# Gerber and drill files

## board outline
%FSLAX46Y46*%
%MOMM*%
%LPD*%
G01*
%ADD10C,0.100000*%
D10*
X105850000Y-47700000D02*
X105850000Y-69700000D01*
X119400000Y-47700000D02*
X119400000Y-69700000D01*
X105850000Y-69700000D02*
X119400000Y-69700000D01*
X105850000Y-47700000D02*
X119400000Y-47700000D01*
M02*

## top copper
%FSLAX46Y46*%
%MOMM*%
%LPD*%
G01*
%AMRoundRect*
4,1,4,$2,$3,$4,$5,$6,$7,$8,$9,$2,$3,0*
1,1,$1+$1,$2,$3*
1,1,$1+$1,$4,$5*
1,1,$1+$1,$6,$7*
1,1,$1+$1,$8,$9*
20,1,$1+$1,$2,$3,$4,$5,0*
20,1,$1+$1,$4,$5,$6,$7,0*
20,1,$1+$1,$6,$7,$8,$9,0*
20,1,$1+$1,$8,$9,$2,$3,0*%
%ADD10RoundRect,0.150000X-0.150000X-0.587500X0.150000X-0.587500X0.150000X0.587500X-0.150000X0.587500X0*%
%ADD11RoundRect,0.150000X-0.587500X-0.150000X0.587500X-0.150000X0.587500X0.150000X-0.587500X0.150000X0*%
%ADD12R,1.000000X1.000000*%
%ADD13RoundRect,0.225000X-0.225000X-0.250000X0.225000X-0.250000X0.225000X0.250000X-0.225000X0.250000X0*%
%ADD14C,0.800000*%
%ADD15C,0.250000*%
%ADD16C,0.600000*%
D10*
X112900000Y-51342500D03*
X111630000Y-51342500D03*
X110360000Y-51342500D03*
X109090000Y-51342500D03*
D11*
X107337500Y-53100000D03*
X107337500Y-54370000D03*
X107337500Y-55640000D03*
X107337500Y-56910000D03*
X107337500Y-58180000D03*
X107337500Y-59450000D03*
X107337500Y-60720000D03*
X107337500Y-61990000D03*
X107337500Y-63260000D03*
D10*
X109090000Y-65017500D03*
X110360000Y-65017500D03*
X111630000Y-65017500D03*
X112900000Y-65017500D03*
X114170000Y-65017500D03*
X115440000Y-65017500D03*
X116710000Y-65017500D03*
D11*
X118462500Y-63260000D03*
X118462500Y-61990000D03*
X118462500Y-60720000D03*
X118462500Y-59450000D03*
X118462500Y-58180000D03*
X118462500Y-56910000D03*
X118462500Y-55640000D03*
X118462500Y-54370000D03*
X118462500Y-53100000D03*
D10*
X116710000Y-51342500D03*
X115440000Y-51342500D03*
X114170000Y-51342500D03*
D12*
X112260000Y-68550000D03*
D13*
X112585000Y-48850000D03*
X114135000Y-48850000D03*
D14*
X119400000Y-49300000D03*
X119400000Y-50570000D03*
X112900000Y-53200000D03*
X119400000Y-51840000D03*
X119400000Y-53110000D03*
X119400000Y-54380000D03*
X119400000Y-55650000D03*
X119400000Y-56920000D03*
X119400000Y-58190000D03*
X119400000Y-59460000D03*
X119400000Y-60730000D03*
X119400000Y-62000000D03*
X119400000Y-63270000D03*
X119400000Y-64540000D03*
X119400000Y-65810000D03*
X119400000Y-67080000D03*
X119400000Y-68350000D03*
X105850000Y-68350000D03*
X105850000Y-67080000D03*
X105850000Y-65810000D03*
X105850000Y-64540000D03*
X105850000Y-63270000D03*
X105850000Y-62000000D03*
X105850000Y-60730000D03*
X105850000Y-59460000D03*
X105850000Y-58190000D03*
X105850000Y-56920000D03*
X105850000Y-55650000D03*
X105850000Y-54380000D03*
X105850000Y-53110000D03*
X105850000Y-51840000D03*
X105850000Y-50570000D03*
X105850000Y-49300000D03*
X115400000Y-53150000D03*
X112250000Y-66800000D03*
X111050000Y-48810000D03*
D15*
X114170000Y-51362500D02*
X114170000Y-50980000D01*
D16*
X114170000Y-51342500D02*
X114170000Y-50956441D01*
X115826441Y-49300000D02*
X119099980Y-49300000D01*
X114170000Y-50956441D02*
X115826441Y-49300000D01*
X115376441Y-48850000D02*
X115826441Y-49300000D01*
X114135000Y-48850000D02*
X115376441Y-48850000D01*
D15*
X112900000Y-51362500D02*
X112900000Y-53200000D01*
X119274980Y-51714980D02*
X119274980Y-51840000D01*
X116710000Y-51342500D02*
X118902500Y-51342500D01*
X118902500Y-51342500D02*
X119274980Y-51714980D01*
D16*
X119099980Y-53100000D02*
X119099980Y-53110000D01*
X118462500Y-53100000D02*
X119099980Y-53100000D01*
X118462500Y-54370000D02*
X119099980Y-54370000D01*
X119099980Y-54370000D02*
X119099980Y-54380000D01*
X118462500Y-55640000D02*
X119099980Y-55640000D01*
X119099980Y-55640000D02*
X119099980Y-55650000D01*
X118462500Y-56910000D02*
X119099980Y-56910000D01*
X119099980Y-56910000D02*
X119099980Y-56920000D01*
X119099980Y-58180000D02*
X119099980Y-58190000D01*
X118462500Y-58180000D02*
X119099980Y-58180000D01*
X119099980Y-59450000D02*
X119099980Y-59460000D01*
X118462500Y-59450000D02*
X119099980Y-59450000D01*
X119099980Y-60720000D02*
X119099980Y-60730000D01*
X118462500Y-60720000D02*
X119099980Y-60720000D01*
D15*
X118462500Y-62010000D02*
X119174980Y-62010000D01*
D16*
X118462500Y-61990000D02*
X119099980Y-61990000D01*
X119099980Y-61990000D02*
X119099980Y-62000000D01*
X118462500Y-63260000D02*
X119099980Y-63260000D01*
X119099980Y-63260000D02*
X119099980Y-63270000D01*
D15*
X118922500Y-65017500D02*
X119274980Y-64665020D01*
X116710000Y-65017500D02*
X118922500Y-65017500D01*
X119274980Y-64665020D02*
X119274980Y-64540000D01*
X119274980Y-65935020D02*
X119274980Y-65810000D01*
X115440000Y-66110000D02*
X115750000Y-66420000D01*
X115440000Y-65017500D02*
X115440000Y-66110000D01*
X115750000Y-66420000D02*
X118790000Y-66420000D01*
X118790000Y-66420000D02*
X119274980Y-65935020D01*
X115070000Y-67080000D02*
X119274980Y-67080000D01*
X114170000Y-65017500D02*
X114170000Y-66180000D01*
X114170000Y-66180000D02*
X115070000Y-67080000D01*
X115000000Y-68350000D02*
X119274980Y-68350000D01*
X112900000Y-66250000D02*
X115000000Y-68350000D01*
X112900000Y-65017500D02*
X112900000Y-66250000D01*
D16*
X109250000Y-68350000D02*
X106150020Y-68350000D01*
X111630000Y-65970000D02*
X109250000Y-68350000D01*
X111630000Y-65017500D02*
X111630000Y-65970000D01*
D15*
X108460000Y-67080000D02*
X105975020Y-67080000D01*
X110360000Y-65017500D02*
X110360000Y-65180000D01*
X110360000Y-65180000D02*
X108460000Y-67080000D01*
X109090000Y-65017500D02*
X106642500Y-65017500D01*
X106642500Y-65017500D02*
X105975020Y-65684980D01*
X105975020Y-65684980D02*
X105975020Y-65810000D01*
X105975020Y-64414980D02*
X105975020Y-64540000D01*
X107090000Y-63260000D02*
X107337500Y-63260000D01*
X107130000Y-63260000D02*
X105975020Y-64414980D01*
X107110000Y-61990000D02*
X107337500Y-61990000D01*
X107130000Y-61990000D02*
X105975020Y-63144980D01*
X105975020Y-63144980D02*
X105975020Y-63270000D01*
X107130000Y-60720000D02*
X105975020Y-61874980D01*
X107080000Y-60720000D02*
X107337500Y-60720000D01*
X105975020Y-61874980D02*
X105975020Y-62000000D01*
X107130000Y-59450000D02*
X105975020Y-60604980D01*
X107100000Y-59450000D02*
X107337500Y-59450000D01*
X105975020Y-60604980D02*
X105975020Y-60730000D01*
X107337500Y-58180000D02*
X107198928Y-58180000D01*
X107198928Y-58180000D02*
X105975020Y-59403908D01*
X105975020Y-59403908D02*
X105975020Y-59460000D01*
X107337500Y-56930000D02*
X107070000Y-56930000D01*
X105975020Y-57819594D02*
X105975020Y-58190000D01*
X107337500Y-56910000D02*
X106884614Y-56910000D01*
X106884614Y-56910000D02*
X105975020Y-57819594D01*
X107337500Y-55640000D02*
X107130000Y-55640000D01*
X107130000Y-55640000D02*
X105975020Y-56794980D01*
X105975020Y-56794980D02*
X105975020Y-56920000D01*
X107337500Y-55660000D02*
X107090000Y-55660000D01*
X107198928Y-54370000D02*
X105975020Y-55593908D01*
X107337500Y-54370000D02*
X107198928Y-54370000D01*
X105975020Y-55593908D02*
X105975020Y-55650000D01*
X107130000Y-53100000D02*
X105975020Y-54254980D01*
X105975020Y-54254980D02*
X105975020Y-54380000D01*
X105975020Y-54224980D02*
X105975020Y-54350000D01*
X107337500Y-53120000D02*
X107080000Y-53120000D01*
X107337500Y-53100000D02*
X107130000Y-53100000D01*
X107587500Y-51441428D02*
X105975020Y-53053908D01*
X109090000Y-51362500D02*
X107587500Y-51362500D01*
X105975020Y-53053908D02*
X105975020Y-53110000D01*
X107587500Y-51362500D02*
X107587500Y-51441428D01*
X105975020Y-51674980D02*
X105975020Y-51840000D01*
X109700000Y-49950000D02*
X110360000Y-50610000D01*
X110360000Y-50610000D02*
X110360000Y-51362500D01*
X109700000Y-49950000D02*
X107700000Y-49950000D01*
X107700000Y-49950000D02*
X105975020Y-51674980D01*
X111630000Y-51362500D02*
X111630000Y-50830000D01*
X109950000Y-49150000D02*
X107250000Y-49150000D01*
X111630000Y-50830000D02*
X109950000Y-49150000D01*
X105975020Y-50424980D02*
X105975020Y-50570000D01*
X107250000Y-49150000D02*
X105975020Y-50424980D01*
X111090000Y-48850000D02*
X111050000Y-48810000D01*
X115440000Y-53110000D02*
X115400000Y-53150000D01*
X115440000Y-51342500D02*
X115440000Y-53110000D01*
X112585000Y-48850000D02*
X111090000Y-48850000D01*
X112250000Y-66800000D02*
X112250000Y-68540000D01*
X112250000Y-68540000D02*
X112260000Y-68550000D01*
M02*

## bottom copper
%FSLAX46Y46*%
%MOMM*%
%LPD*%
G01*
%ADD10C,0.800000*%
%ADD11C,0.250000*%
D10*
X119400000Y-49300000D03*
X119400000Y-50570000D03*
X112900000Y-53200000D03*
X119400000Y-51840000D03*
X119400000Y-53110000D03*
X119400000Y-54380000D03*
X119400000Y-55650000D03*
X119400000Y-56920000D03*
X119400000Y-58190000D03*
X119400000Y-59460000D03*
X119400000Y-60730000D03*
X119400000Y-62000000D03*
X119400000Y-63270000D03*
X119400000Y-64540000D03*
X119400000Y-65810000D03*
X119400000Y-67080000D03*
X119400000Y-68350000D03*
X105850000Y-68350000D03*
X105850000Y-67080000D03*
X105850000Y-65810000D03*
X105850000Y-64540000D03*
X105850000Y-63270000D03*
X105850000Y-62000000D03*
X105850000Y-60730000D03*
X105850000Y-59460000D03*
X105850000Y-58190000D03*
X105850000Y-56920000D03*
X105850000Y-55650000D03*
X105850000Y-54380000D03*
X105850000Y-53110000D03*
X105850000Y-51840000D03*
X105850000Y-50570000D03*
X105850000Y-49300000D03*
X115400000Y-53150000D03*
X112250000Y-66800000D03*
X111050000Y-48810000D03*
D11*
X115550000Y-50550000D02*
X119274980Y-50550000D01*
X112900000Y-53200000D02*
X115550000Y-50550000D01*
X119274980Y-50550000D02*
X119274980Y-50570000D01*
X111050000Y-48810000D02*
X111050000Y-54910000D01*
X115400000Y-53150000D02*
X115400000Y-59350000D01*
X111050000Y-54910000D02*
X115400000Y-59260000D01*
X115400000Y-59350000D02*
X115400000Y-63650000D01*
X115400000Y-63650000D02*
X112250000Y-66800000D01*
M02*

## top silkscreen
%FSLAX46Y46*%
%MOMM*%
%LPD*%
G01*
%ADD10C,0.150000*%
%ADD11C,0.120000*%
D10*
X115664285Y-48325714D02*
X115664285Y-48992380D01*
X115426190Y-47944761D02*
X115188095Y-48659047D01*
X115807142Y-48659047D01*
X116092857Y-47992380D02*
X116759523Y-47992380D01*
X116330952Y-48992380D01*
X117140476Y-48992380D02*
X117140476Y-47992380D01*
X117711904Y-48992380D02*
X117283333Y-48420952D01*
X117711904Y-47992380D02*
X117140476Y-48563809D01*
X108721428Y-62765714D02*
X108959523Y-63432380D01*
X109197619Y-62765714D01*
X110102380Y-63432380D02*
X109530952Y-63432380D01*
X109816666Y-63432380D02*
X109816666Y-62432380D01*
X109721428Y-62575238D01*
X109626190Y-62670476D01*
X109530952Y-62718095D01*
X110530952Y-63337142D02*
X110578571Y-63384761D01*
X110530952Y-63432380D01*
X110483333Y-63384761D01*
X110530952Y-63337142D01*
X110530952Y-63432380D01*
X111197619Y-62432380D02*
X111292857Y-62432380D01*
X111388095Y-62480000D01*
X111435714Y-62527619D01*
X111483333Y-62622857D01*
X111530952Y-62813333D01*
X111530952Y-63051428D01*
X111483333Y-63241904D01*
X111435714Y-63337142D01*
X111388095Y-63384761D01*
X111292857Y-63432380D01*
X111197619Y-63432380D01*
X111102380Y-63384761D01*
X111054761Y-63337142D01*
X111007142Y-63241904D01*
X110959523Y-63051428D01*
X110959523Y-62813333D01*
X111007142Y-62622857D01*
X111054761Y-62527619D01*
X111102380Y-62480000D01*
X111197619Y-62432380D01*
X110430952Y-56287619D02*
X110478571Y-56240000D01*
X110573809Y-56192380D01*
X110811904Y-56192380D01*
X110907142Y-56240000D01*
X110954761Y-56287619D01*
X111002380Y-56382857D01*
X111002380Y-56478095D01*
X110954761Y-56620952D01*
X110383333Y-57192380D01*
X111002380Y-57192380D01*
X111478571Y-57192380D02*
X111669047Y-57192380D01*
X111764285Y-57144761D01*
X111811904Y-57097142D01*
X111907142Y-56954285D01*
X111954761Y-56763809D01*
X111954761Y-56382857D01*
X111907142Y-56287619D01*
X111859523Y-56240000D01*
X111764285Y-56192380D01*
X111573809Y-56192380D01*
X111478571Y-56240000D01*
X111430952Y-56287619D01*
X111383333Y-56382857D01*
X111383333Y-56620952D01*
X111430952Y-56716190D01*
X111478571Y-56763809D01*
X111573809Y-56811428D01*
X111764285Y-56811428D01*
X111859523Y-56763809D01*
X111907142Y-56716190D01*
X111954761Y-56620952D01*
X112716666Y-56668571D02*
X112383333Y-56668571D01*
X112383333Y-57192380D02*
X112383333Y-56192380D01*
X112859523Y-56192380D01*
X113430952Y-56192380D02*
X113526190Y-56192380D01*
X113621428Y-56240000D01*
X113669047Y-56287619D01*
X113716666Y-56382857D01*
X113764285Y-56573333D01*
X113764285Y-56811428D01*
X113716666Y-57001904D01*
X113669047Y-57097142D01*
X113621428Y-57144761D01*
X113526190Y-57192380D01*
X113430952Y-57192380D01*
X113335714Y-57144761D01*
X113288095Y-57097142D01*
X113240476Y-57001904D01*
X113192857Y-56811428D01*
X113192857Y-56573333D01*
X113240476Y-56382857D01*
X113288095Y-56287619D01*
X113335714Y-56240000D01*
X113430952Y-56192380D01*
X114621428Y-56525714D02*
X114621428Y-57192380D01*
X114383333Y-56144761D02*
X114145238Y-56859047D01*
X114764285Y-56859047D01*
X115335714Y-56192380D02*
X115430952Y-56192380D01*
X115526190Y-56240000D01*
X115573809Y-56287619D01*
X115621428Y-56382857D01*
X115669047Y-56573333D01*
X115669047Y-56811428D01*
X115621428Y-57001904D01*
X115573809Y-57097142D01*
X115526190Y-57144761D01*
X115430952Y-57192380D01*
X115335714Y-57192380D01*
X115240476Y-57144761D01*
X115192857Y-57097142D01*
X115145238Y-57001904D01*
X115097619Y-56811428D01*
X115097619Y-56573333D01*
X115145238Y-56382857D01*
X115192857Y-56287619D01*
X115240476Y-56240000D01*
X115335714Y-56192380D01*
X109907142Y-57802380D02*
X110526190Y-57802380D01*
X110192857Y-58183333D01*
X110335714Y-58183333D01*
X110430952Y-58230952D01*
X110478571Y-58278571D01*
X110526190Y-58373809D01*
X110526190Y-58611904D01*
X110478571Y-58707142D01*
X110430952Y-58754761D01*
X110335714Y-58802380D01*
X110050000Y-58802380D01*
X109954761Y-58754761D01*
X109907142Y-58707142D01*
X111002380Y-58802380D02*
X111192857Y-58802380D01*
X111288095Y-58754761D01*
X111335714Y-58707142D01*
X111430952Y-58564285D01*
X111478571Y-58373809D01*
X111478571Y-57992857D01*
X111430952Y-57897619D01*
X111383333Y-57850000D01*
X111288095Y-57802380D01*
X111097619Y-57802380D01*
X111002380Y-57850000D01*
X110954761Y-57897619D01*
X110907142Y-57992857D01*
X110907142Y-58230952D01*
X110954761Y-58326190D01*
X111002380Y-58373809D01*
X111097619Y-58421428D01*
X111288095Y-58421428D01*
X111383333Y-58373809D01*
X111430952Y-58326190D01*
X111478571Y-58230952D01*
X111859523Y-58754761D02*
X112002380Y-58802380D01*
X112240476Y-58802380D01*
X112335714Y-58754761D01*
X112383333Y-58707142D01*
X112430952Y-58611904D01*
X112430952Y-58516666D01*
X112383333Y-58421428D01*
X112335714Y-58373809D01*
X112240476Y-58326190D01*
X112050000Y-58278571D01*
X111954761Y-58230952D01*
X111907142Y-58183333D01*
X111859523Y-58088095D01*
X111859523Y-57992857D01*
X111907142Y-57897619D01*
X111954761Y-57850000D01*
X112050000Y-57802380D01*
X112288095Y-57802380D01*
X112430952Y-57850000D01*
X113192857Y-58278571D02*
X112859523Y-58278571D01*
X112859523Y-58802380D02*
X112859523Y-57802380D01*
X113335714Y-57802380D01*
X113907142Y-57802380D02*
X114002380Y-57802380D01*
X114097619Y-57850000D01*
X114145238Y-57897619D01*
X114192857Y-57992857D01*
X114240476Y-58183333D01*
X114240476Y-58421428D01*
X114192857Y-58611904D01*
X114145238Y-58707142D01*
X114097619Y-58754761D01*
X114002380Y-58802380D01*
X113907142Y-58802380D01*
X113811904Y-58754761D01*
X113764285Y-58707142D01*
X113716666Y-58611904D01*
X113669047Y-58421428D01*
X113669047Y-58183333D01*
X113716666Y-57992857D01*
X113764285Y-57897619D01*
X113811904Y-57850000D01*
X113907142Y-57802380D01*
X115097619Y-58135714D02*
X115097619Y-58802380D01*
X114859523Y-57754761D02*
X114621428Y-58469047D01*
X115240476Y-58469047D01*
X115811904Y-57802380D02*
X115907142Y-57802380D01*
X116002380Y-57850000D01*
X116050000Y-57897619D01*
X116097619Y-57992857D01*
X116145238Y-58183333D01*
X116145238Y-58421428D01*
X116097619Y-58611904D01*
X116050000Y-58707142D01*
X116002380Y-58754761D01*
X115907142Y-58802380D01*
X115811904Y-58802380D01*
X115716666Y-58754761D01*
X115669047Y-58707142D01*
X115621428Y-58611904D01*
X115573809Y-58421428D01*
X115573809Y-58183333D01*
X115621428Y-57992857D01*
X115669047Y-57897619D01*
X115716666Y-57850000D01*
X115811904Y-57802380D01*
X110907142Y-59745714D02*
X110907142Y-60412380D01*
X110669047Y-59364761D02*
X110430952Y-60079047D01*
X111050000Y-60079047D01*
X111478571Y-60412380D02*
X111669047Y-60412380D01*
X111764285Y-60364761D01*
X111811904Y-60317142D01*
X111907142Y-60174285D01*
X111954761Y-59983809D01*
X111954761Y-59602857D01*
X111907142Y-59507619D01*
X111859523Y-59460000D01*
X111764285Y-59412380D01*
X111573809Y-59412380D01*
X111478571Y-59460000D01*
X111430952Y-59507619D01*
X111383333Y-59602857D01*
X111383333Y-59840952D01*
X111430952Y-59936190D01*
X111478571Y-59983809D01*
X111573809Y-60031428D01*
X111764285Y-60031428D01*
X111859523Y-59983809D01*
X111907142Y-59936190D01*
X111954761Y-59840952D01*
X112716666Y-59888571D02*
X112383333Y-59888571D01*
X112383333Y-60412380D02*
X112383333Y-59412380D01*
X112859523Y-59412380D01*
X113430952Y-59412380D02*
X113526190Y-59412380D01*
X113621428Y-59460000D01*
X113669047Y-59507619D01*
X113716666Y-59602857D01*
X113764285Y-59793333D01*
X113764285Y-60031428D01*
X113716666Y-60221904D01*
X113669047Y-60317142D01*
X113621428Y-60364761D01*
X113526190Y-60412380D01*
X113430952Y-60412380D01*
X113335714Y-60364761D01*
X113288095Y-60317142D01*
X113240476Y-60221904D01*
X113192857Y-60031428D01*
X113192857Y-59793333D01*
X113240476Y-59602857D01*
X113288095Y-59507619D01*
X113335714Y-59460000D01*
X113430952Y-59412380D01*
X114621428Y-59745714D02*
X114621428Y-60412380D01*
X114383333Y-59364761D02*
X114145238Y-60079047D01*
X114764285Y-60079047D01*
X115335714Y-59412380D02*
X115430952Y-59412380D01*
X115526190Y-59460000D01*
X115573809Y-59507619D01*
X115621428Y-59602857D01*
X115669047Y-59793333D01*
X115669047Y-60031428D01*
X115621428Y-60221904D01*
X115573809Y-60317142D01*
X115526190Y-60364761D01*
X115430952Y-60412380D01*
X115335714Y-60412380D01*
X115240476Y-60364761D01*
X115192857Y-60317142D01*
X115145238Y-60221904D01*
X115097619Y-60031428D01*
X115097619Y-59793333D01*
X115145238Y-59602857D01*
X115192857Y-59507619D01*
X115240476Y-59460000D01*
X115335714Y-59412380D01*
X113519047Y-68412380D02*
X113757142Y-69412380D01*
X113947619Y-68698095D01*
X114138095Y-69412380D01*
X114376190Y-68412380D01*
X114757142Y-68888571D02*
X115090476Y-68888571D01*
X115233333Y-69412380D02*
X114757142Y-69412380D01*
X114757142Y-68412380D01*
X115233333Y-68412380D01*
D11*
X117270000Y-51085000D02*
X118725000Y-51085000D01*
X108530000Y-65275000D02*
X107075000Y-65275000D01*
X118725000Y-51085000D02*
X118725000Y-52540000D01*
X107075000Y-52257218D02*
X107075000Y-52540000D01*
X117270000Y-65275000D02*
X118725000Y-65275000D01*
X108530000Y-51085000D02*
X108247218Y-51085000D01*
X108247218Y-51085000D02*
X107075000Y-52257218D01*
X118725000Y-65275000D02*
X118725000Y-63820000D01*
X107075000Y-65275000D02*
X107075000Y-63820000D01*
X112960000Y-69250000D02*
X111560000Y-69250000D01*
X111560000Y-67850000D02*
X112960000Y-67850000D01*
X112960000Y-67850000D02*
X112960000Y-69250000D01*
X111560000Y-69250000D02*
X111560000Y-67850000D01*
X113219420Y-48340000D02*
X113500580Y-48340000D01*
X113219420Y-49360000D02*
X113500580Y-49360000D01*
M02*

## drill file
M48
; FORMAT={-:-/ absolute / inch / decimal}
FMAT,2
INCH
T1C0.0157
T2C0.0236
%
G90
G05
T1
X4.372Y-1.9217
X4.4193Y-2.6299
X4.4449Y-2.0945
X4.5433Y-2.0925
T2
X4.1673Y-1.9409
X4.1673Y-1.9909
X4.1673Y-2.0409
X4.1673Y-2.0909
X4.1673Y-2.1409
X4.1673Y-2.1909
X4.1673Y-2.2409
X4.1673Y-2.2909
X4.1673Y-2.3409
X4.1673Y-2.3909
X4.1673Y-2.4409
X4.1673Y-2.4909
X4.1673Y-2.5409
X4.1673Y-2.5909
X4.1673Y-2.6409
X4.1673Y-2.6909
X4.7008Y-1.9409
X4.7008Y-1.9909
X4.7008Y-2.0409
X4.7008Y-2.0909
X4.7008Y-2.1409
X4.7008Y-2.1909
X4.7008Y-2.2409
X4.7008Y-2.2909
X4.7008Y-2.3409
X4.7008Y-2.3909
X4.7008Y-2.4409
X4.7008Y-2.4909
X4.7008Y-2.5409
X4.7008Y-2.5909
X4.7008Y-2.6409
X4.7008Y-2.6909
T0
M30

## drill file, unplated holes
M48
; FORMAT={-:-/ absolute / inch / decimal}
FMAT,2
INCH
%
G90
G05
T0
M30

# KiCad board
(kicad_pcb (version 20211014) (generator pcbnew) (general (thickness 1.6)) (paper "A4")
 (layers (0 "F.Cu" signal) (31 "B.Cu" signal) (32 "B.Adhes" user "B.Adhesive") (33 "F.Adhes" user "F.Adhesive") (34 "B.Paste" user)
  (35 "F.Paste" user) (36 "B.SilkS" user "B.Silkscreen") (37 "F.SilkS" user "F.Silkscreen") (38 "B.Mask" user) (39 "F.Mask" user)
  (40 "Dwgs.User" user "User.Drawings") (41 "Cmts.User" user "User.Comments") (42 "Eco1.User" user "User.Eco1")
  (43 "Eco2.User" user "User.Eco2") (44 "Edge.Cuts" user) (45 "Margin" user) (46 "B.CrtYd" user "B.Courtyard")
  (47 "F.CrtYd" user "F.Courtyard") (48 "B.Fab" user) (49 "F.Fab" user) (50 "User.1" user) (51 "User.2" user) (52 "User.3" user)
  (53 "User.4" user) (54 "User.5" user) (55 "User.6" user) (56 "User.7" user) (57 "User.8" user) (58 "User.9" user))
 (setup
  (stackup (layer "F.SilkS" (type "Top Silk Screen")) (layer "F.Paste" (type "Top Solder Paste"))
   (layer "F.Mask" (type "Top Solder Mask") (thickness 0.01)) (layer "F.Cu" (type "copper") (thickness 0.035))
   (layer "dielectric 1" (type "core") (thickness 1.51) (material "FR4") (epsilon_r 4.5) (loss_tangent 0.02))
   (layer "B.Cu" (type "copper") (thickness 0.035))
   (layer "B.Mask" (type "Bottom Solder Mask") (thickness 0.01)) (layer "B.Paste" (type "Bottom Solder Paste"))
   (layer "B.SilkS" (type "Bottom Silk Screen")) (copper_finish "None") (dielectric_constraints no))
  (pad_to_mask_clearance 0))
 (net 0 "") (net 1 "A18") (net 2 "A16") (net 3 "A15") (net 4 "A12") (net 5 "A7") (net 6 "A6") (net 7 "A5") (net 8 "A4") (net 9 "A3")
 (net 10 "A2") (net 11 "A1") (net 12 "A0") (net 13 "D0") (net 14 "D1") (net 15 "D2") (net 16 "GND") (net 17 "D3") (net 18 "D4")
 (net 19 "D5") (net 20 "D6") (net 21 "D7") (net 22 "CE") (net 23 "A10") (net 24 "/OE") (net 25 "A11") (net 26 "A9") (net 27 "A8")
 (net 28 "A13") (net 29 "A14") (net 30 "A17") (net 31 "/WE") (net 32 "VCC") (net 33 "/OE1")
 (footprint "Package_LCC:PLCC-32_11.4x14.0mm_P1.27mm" (layer "F.Cu") (at 112.9 58.18)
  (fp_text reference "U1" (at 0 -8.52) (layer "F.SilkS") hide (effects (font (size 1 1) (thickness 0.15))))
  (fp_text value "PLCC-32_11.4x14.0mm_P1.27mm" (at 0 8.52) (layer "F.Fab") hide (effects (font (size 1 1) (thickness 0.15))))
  (fp_line (start 4.37 -7.095) (end 5.825 -7.095) (layer "F.SilkS") (width 0.12))
  (fp_line (start -4.37 7.095) (end -5.825 7.095) (layer "F.SilkS") (width 0.12))
  (fp_line (start 5.825 -7.095) (end 5.825 -5.64) (layer "F.SilkS") (width 0.12))
  (fp_line (start -5.825 -5.922782) (end -5.825 -5.64) (layer "F.SilkS") (width 0.12))
  (fp_line (start 4.37 7.095) (end 5.825 7.095) (layer "F.SilkS") (width 0.12))
  (fp_line (start -4.37 -7.095) (end -4.652782 -7.095) (layer "F.SilkS") (width 0.12))
  (fp_line (start -4.652782 -7.095) (end -5.825 -5.922782) (layer "F.SilkS") (width 0.12))
  (fp_line (start 5.825 7.095) (end 5.825 5.64) (layer "F.SilkS") (width 0.12))
  (fp_line (start -5.825 7.095) (end -5.825 5.64) (layer "F.SilkS") (width 0.12))
  (pad "1" smd roundrect (at 0 -6.8375) (size 0.6 1.475) (layers "F.Cu" "F.Paste" "F.Mask") (roundrect_rratio 0.25) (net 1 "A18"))
  (pad "2" smd roundrect (at -1.27 -6.8375) (size 0.6 1.475) (layers "F.Cu" "F.Paste" "F.Mask") (roundrect_rratio 0.25) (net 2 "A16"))
  (pad "3" smd roundrect (at -2.54 -6.8375) (size 0.6 1.475) (layers "F.Cu" "F.Paste" "F.Mask") (roundrect_rratio 0.25) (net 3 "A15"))
  (pad "4" smd roundrect (at -3.81 -6.8375) (size 0.6 1.475) (layers "F.Cu" "F.Paste" "F.Mask") (roundrect_rratio 0.25) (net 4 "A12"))
  (pad "5" smd roundrect (at -5.5625 -5.08) (size 1.475 0.6) (layers "F.Cu" "F.Paste" "F.Mask") (roundrect_rratio 0.25) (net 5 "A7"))
  (pad "6" smd roundrect (at -5.5625 -3.81) (size 1.475 0.6) (layers "F.Cu" "F.Paste" "F.Mask") (roundrect_rratio 0.25) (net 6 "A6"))
  (pad "7" smd roundrect (at -5.5625 -2.54) (size 1.475 0.6) (layers "F.Cu" "F.Paste" "F.Mask") (roundrect_rratio 0.25) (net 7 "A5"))
  (pad "8" smd roundrect (at -5.5625 -1.27) (size 1.475 0.6) (layers "F.Cu" "F.Paste" "F.Mask") (roundrect_rratio 0.25) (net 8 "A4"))
  (pad "9" smd roundrect (at -5.5625 0) (size 1.475 0.6) (layers "F.Cu" "F.Paste" "F.Mask") (roundrect_rratio 0.25) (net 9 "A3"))
  (pad "10" smd roundrect (at -5.5625 1.27) (size 1.475 0.6) (layers "F.Cu" "F.Paste" "F.Mask") (roundrect_rratio 0.25) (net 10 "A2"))
  (pad "11" smd roundrect (at -5.5625 2.54) (size 1.475 0.6) (layers "F.Cu" "F.Paste" "F.Mask") (roundrect_rratio 0.25) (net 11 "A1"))
  (pad "12" smd roundrect (at -5.5625 3.81) (size 1.475 0.6) (layers "F.Cu" "F.Paste" "F.Mask") (roundrect_rratio 0.25) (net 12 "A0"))
  (pad "13" smd roundrect (at -5.5625 5.08) (size 1.475 0.6) (layers "F.Cu" "F.Paste" "F.Mask") (roundrect_rratio 0.25) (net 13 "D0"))
  (pad "14" smd roundrect (at -3.81 6.8375) (size 0.6 1.475) (layers "F.Cu" "F.Paste" "F.Mask") (roundrect_rratio 0.25) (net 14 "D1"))
  (pad "15" smd roundrect (at -2.54 6.8375) (size 0.6 1.475) (layers "F.Cu" "F.Paste" "F.Mask") (roundrect_rratio 0.25) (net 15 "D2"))
  (pad "16" smd roundrect (at -1.27 6.8375) (size 0.6 1.475) (layers "F.Cu" "F.Paste" "F.Mask") (roundrect_rratio 0.25) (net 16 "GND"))
  (pad "17" smd roundrect (at 0 6.8375) (size 0.6 1.475) (layers "F.Cu" "F.Paste" "F.Mask") (roundrect_rratio 0.25) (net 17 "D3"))
  (pad "18" smd roundrect (at 1.27 6.8375) (size 0.6 1.475) (layers "F.Cu" "F.Paste" "F.Mask") (roundrect_rratio 0.25) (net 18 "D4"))
  (pad "19" smd roundrect (at 2.54 6.8375) (size 0.6 1.475) (layers "F.Cu" "F.Paste" "F.Mask") (roundrect_rratio 0.25) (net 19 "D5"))
  (pad "20" smd roundrect (at 3.81 6.8375) (size 0.6 1.475) (layers "F.Cu" "F.Paste" "F.Mask") (roundrect_rratio 0.25) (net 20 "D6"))
  (pad "21" smd roundrect (at 5.5625 5.08) (size 1.475 0.6) (layers "F.Cu" "F.Paste" "F.Mask") (roundrect_rratio 0.25) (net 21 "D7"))
  (pad "22" smd roundrect (at 5.5625 3.81) (size 1.475 0.6) (layers "F.Cu" "F.Paste" "F.Mask") (roundrect_rratio 0.25) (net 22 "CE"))
  (pad "23" smd roundrect (at 5.5625 2.54) (size 1.475 0.6) (layers "F.Cu" "F.Paste" "F.Mask") (roundrect_rratio 0.25) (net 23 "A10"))
  (pad "24" smd roundrect (at 5.5625 1.27) (size 1.475 0.6) (layers "F.Cu" "F.Paste" "F.Mask") (roundrect_rratio 0.25) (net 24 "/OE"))
  (pad "25" smd roundrect (at 5.5625 0) (size 1.475 0.6) (layers "F.Cu" "F.Paste" "F.Mask") (roundrect_rratio 0.25) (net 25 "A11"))
  (pad "26" smd roundrect (at 5.5625 -1.27) (size 1.475 0.6) (layers "F.Cu" "F.Paste" "F.Mask") (roundrect_rratio 0.25) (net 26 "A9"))
  (pad "27" smd roundrect (at 5.5625 -2.54) (size 1.475 0.6) (layers "F.Cu" "F.Paste" "F.Mask") (roundrect_rratio 0.25) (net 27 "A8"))
  (pad "28" smd roundrect (at 5.5625 -3.81) (size 1.475 0.6) (layers "F.Cu" "F.Paste" "F.Mask") (roundrect_rratio 0.25) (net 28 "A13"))
  (pad "29" smd roundrect (at 5.5625 -5.08) (size 1.475 0.6) (layers "F.Cu" "F.Paste" "F.Mask") (roundrect_rratio 0.25) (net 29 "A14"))
  (pad "30" smd roundrect (at 3.81 -6.8375) (size 0.6 1.475) (layers "F.Cu" "F.Paste" "F.Mask") (roundrect_rratio 0.25) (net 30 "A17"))
  (pad "31" smd roundrect (at 2.54 -6.8375) (size 0.6 1.475) (layers "F.Cu" "F.Paste" "F.Mask") (roundrect_rratio 0.25) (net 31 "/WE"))
  (pad "32" smd roundrect (at 1.27 -6.8375) (size 0.6 1.475) (layers "F.Cu" "F.Paste" "F.Mask") (roundrect_rratio 0.25) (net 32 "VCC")))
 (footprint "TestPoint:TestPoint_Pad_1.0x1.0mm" (layer "F.Cu") (at 112.26 68.55)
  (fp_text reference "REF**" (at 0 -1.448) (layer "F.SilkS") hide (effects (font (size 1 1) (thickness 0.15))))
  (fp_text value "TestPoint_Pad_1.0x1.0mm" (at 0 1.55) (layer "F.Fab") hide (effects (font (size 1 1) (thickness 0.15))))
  (fp_line (start 0.7 0.7) (end -0.7 0.7) (layer "F.SilkS") (width 0.12))
  (fp_line (start -0.7 -0.7) (end 0.7 -0.7) (layer "F.SilkS") (width 0.12))
  (fp_line (start 0.7 -0.7) (end 0.7 0.7) (layer "F.SilkS") (width 0.12))
  (fp_line (start -0.7 0.7) (end -0.7 -0.7) (layer "F.SilkS") (width 0.12))
  (pad "1" smd rect (at 0 0) (size 1 1) (layers "F.Cu" "F.Mask") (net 31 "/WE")))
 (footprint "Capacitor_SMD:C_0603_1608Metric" (layer "F.Cu") (at 113.36 48.85)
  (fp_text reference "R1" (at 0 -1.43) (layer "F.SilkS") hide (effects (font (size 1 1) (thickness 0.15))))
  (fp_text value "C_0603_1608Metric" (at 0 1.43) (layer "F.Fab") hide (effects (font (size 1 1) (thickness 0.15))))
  (fp_line (start -0.14058 -0.51) (end 0.14058 -0.51) (layer "F.SilkS") (width 0.12))
  (fp_line (start -0.14058 0.51) (end 0.14058 0.51) (layer "F.SilkS") (width 0.12))
  (pad "1" smd roundrect (at -0.775 0) (size 0.9 0.95) (layers "F.Cu" "F.Paste" "F.Mask") (roundrect_rratio 0.25) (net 31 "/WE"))
  (pad "2" smd roundrect (at 0.775 0) (size 0.9 0.95) (layers "F.Cu" "F.Paste" "F.Mask") (roundrect_rratio 0.25) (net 32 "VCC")))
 (gr_line (start 105.85 47.7) (end 105.85 69.7) (layer "Edge.Cuts") (width 0.1))
 (gr_line (start 119.4 47.7) (end 119.4 69.7) (layer "Edge.Cuts") (width 0.1))
 (gr_line (start 105.85 69.7) (end 119.4 69.7) (layer "Edge.Cuts") (width 0.1))
 (gr_line (start 105.85 47.7) (end 119.4 47.7) (layer "Edge.Cuts") (width 0.1))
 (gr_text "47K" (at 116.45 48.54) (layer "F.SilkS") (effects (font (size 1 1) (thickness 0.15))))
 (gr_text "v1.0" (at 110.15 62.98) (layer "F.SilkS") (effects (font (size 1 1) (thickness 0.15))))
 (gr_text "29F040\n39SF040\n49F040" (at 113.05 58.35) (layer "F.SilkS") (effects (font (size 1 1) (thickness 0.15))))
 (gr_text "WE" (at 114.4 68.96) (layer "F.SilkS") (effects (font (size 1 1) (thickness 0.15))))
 (segment (start 114.17 51.3625) (end 114.17 50.98) (width 0.25) (layer "F.Cu") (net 32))
 (segment (start 114.17 51.3425) (end 114.17 50.956441) (width 0.6) (layer "F.Cu") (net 32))
 (segment (start 115.826441 49.3) (end 119.09998 49.3) (width 0.6) (layer "F.Cu") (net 32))
 (segment (start 114.17 50.956441) (end 115.826441 49.3) (width 0.6) (layer "F.Cu") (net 32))
 (segment (start 115.376441 48.85) (end 115.826441 49.3) (width 0.6) (layer "F.Cu") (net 32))
 (segment (start 114.135 48.85) (end 115.376441 48.85) (width 0.6) (layer "F.Cu") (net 32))
 (via (at 119.4 49.3) (size 0.8) (drill 0.6) (layers "F.Cu" "B.Cu") (free) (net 32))
 (segment (start 112.9 51.3625) (end 112.9 53.2) (width 0.25) (layer "F.Cu") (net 1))
 (via (at 119.4 50.57) (size 0.8) (drill 0.6) (layers "F.Cu" "B.Cu") (free) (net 1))
 (via (at 112.9 53.2) (size 0.8) (drill 0.4) (layers "F.Cu" "B.Cu") (free) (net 1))
 (segment (start 115.55 50.55) (end 119.27498 50.55) (width 0.25) (layer "B.Cu") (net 1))
 (segment (start 112.9 53.2) (end 115.55 50.55) (width 0.25) (layer "B.Cu") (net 1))
 (segment (start 119.27498 50.55) (end 119.27498 50.57) (width 0.25) (layer "B.Cu") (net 1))
 (segment (start 119.27498 51.71498) (end 119.27498 51.84) (width 0.25) (layer "F.Cu") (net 30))
 (segment (start 116.71 51.3425) (end 118.9025 51.3425) (width 0.25) (layer "F.Cu") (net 30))
 (segment (start 118.9025 51.3425) (end 119.27498 51.71498) (width 0.25) (layer "F.Cu") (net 30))
 (via (at 119.4 51.84) (size 0.8) (drill 0.6) (layers "F.Cu" "B.Cu") (free) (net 30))
 (segment (start 119.09998 53.1) (end 119.09998 53.11) (width 0.6) (layer "F.Cu") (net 29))
 (segment (start 118.4625 53.1) (end 119.09998 53.1) (width 0.6) (layer "F.Cu") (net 29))
 (via (at 119.4 53.11) (size 0.8) (drill 0.6) (layers "F.Cu" "B.Cu") (free) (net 29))
 (segment (start 118.4625 54.37) (end 119.09998 54.37) (width 0.6) (layer "F.Cu") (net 28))
 (segment (start 119.09998 54.37) (end 119.09998 54.38) (width 0.6) (layer "F.Cu") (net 28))
 (via (at 119.4 54.38) (size 0.8) (drill 0.6) (layers "F.Cu" "B.Cu") (free) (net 28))
 (segment (start 118.4625 55.64) (end 119.09998 55.64) (width 0.6) (layer "F.Cu") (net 27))
 (segment (start 119.09998 55.64) (end 119.09998 55.65) (width 0.6) (layer "F.Cu") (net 27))
 (via (at 119.4 55.65) (size 0.8) (drill 0.6) (layers "F.Cu" "B.Cu") (free) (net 27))
 (segment (start 118.4625 56.91) (end 119.09998 56.91) (width 0.6) (layer "F.Cu") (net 26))
 (segment (start 119.09998 56.91) (end 119.09998 56.92) (width 0.6) (layer "F.Cu") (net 26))
 (via (at 119.4 56.92) (size 0.8) (drill 0.6) (layers "F.Cu" "B.Cu") (free) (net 26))
 (segment (start 119.09998 58.18) (end 119.09998 58.19) (width 0.6) (layer "F.Cu") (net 25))
 (segment (start 118.4625 58.18) (end 119.09998 58.18) (width 0.6) (layer "F.Cu") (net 25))
 (via (at 119.4 58.19) (size 0.8) (drill 0.6) (layers "F.Cu" "B.Cu") (free) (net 25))
 (segment (start 119.09998 59.45) (end 119.09998 59.46) (width 0.6) (layer "F.Cu") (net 24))
 (segment (start 118.4625 59.45) (end 119.09998 59.45) (width 0.6) (layer "F.Cu") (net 24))
 (via (at 119.4 59.46) (size 0.8) (drill 0.6) (layers "F.Cu" "B.Cu") (free) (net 24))
 (segment (start 119.09998 60.72) (end 119.09998 60.73) (width 0.6) (layer "F.Cu") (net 23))
 (segment (start 118.4625 60.72) (end 119.09998 60.72) (width 0.6) (layer "F.Cu") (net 23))
 (via (at 119.4 60.73) (size 0.8) (drill 0.6) (layers "F.Cu" "B.Cu") (free) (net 23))
 (segment (start 118.4625 62.01) (end 119.17498 62.01) (width 0.25) (layer "F.Cu") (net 22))
 (segment (start 118.4625 61.99) (end 119.09998 61.99) (width 0.6) (layer "F.Cu") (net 22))
 (segment (start 119.09998 61.99) (end 119.09998 62) (width 0.6) (layer "F.Cu") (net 22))
 (via (at 119.4 62) (size 0.8) (drill 0.6) (layers "F.Cu" "B.Cu") (free) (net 22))
 (segment (start 118.4625 63.26) (end 119.09998 63.26) (width 0.6) (layer "F.Cu") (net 21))
 (segment (start 119.09998 63.26) (end 119.09998 63.27) (width 0.6) (layer "F.Cu") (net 21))
 (via (at 119.4 63.27) (size 0.8) (drill 0.6) (layers "F.Cu" "B.Cu") (free) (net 21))
 (segment (start 118.9225 65.0175) (end 119.27498 64.66502) (width 0.25) (layer "F.Cu") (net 20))
 (segment (start 116.71 65.0175) (end 118.9225 65.0175) (width 0.25) (layer "F.Cu") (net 20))
 (segment (start 119.27498 64.66502) (end 119.27498 64.54) (width 0.25) (layer "F.Cu") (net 20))
 (via (at 119.4 64.54) (size 0.8) (drill 0.6) (layers "F.Cu" "B.Cu") (free) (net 20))
 (segment (start 119.27498 65.93502) (end 119.27498 65.81) (width 0.25) (layer "F.Cu") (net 19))
 (segment (start 115.44 66.11) (end 115.75 66.42) (width 0.25) (layer "F.Cu") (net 19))
 (segment (start 115.44 65.0175) (end 115.44 66.11) (width 0.25) (layer "F.Cu") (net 19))
 (segment (start 115.75 66.42) (end 118.79 66.42) (width 0.25) (layer "F.Cu") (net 19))
 (segment (start 118.79 66.42) (end 119.27498 65.93502) (width 0.25) (layer "F.Cu") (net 19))
 (via (at 119.4 65.81) (size 0.8) (drill 0.6) (layers "F.Cu" "B.Cu") (free) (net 19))
 (segment (start 115.07 67.08) (end 119.27498 67.08) (width 0.25) (layer "F.Cu") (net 18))
 (segment (start 114.17 65.0175) (end 114.17 66.18) (width 0.25) (layer "F.Cu") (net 18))
 (segment (start 114.17 66.18) (end 115.07 67.08) (width 0.25) (layer "F.Cu") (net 18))
 (via (at 119.4 67.08) (size 0.8) (drill 0.6) (layers "F.Cu" "B.Cu") (free) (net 18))
 (segment (start 115 68.35) (end 119.27498 68.35) (width 0.25) (layer "F.Cu") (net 17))
 (segment (start 112.9 66.25) (end 115 68.35) (width 0.25) (layer "F.Cu") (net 17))
 (segment (start 112.9 65.0175) (end 112.9 66.25) (width 0.25) (layer "F.Cu") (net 17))
 (via (at 119.4 68.35) (size 0.8) (drill 0.6) (layers "F.Cu" "B.Cu") (free) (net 17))
 (segment (start 109.25 68.35) (end 106.15002 68.35) (width 0.6) (layer "F.Cu") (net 16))
 (segment (start 111.63 65.97) (end 109.25 68.35) (width 0.6) (layer "F.Cu") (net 16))
 (segment (start 111.63 65.0175) (end 111.63 65.97) (width 0.6) (layer "F.Cu") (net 16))
 (via (at 105.85 68.35) (size 0.8) (drill 0.6) (layers "F.Cu" "B.Cu") (free) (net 16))
 (segment (start 108.46 67.08) (end 105.97502 67.08) (width 0.25) (layer "F.Cu") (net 15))
 (segment (start 110.36 65.0175) (end 110.36 65.18) (width 0.25) (layer "F.Cu") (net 15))
 (segment (start 110.36 65.18) (end 108.46 67.08) (width 0.25) (layer "F.Cu") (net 15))
 (via (at 105.85 67.08) (size 0.8) (drill 0.6) (layers "F.Cu" "B.Cu") (free) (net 15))
 (segment (start 109.09 65.0175) (end 106.6425 65.0175) (width 0.25) (layer "F.Cu") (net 14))
 (segment (start 106.6425 65.0175) (end 105.97502 65.68498) (width 0.25) (layer "F.Cu") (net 14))
 (segment (start 105.97502 65.68498) (end 105.97502 65.81) (width 0.25) (layer "F.Cu") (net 14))
 (via (at 105.85 65.81) (size 0.8) (drill 0.6) (layers "F.Cu" "B.Cu") (free) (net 14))
 (segment (start 105.97502 64.41498) (end 105.97502 64.54) (width 0.25) (layer "F.Cu") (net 13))
 (segment (start 107.09 63.26) (end 107.3375 63.26) (width 0.25) (layer "F.Cu") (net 13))
 (segment (start 107.13 63.26) (end 105.97502 64.41498) (width 0.25) (layer "F.Cu") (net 13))
 (via (at 105.85 64.54) (size 0.8) (drill 0.6) (layers "F.Cu" "B.Cu") (free) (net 13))
 (segment (start 107.11 61.99) (end 107.3375 61.99) (width 0.25) (layer "F.Cu") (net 12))
 (segment (start 107.13 61.99) (end 105.97502 63.14498) (width 0.25) (layer "F.Cu") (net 12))
 (segment (start 105.97502 63.14498) (end 105.97502 63.27) (width 0.25) (layer "F.Cu") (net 12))
 (via (at 105.85 63.27) (size 0.8) (drill 0.6) (layers "F.Cu" "B.Cu") (free) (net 12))
 (segment (start 107.13 60.72) (end 105.97502 61.87498) (width 0.25) (layer "F.Cu") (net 11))
 (segment (start 107.08 60.72) (end 107.3375 60.72) (width 0.25) (layer "F.Cu") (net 11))
 (segment (start 105.97502 61.87498) (end 105.97502 62) (width 0.25) (layer "F.Cu") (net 11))
 (via (at 105.85 62) (size 0.8) (drill 0.6) (layers "F.Cu" "B.Cu") (free) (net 11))
 (segment (start 107.13 59.45) (end 105.97502 60.60498) (width 0.25) (layer "F.Cu") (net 10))
 (segment (start 107.1 59.45) (end 107.3375 59.45) (width 0.25) (layer "F.Cu") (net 10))
 (segment (start 105.97502 60.60498) (end 105.97502 60.73) (width 0.25) (layer "F.Cu") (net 10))
 (via (at 105.85 60.73) (size 0.8) (drill 0.6) (layers "F.Cu" "B.Cu") (free) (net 10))
 (segment (start 107.3375 58.18) (end 107.198928 58.18) (width 0.25) (layer "F.Cu") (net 9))
 (segment (start 107.198928 58.18) (end 105.97502 59.403908) (width 0.25) (layer "F.Cu") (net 9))
 (segment (start 105.97502 59.403908) (end 105.97502 59.46) (width 0.25) (layer "F.Cu") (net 9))
 (via (at 105.85 59.46) (size 0.8) (drill 0.6) (layers "F.Cu" "B.Cu") (free) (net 9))
 (segment (start 107.3375 56.93) (end 107.07 56.93) (width 0.25) (layer "F.Cu") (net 8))
 (segment (start 105.97502 57.819594) (end 105.97502 58.19) (width 0.25) (layer "F.Cu") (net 8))
 (segment (start 107.3375 56.91) (end 106.884614 56.91) (width 0.25) (layer "F.Cu") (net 8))
 (segment (start 106.884614 56.91) (end 105.97502 57.819594) (width 0.25) (layer "F.Cu") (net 8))
 (via (at 105.85 58.19) (size 0.8) (drill 0.6) (layers "F.Cu" "B.Cu") (free) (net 8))
 (segment (start 107.3375 55.64) (end 107.13 55.64) (width 0.25) (layer "F.Cu") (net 7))
 (segment (start 107.13 55.64) (end 105.97502 56.79498) (width 0.25) (layer "F.Cu") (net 7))
 (segment (start 105.97502 56.79498) (end 105.97502 56.92) (width 0.25) (layer "F.Cu") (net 7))
 (segment (start 107.3375 55.66) (end 107.09 55.66) (width 0.25) (layer "F.Cu") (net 7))
 (via (at 105.85 56.92) (size 0.8) (drill 0.6) (layers "F.Cu" "B.Cu") (free) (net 7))
 (segment (start 107.198928 54.37) (end 105.97502 55.593908) (width 0.25) (layer "F.Cu") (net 6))
 (segment (start 107.3375 54.37) (end 107.198928 54.37) (width 0.25) (layer "F.Cu") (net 6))
 (segment (start 105.97502 55.593908) (end 105.97502 55.65) (width 0.25) (layer "F.Cu") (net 6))
 (via (at 105.85 55.65) (size 0.8) (drill 0.6) (layers "F.Cu" "B.Cu") (free) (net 6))
 (segment (start 107.13 53.1) (end 105.97502 54.25498) (width 0.25) (layer "F.Cu") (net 5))
 (segment (start 105.97502 54.25498) (end 105.97502 54.38) (width 0.25) (layer "F.Cu") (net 5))
 (segment (start 105.97502 54.22498) (end 105.97502 54.35) (width 0.25) (layer "F.Cu") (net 5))
 (segment (start 107.3375 53.12) (end 107.08 53.12) (width 0.25) (layer "F.Cu") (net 5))
 (segment (start 107.3375 53.1) (end 107.13 53.1) (width 0.25) (layer "F.Cu") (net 5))
 (via (at 105.85 54.38) (size 0.8) (drill 0.6) (layers "F.Cu" "B.Cu") (free) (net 5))
 (segment (start 107.5875 51.441428) (end 105.97502 53.053908) (width 0.25) (layer "F.Cu") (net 4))
 (segment (start 109.09 51.3625) (end 107.5875 51.3625) (width 0.25) (layer "F.Cu") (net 4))
 (segment (start 105.97502 53.053908) (end 105.97502 53.11) (width 0.25) (layer "F.Cu") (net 4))
 (segment (start 107.5875 51.3625) (end 107.5875 51.441428) (width 0.25) (layer "F.Cu") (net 4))
 (via (at 105.85 53.11) (size 0.8) (drill 0.6) (layers "F.Cu" "B.Cu") (free) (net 4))
 (segment (start 105.97502 51.67498) (end 105.97502 51.84) (width 0.25) (layer "F.Cu") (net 3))
 (segment (start 109.7 49.95) (end 110.36 50.61) (width 0.25) (layer "F.Cu") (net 3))
 (segment (start 110.36 50.61) (end 110.36 51.3625) (width 0.25) (layer "F.Cu") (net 3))
 (segment (start 109.7 49.95) (end 107.7 49.95) (width 0.25) (layer "F.Cu") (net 3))
 (segment (start 107.7 49.95) (end 105.97502 51.67498) (width 0.25) (layer "F.Cu") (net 3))
 (via (at 105.85 51.84) (size 0.8) (drill 0.6) (layers "F.Cu" "B.Cu") (free) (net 3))
 (segment (start 111.63 51.3625) (end 111.63 50.83) (width 0.25) (layer "F.Cu") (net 2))
 (segment (start 109.95 49.15) (end 107.25 49.15) (width 0.25) (layer "F.Cu") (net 2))
 (segment (start 111.63 50.83) (end 109.95 49.15) (width 0.25) (layer "F.Cu") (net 2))
 (segment (start 105.97502 50.42498) (end 105.97502 50.57) (width 0.25) (layer "F.Cu") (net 2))
 (segment (start 107.25 49.15) (end 105.97502 50.42498) (width 0.25) (layer "F.Cu") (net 2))
 (via (at 105.85 50.57) (size 0.8) (drill 0.6) (layers "F.Cu" "B.Cu") (free) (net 2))
 (via (at 105.85 49.3) (size 0.8) (drill 0.6) (layers "F.Cu" "B.Cu") (free) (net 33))
 (segment (start 111.09 48.85) (end 111.05 48.81) (width 0.25) (layer "F.Cu") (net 31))
 (segment (start 115.44 53.11) (end 115.4 53.15) (width 0.25) (layer "F.Cu") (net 31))
 (segment (start 115.44 51.3425) (end 115.44 53.11) (width 0.25) (layer "F.Cu") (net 31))
 (segment (start 112.585 48.85) (end 111.09 48.85) (width 0.25) (layer "F.Cu") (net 31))
 (segment (start 112.25 66.8) (end 112.25 68.54) (width 0.25) (layer "F.Cu") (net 31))
 (segment (start 112.25 68.54) (end 112.26 68.55) (width 0.25) (layer "F.Cu") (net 31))
 (via (at 115.4 53.15) (size 0.8) (drill 0.4) (layers "F.Cu" "B.Cu") (free) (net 31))
 (via (at 112.25 66.8) (size 0.8) (drill 0.4) (layers "F.Cu" "B.Cu") (free) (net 31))
 (via (at 111.05 48.81) (size 0.8) (drill 0.4) (layers "F.Cu" "B.Cu") (free) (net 31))
 (segment (start 111.05 48.81) (end 111.05 54.91) (width 0.25) (layer "B.Cu") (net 31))
 (segment (start 115.4 53.15) (end 115.4 59.35) (width 0.25) (layer "B.Cu") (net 31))
 (segment (start 111.05 54.91) (end 115.4 59.26) (width 0.25) (layer "B.Cu") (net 31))
 (segment (start 115.4 59.35) (end 115.4 63.65) (width 0.25) (layer "B.Cu") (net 31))
 (segment (start 115.4 63.65) (end 112.25 66.8) (width 0.25) (layer "B.Cu") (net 31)))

